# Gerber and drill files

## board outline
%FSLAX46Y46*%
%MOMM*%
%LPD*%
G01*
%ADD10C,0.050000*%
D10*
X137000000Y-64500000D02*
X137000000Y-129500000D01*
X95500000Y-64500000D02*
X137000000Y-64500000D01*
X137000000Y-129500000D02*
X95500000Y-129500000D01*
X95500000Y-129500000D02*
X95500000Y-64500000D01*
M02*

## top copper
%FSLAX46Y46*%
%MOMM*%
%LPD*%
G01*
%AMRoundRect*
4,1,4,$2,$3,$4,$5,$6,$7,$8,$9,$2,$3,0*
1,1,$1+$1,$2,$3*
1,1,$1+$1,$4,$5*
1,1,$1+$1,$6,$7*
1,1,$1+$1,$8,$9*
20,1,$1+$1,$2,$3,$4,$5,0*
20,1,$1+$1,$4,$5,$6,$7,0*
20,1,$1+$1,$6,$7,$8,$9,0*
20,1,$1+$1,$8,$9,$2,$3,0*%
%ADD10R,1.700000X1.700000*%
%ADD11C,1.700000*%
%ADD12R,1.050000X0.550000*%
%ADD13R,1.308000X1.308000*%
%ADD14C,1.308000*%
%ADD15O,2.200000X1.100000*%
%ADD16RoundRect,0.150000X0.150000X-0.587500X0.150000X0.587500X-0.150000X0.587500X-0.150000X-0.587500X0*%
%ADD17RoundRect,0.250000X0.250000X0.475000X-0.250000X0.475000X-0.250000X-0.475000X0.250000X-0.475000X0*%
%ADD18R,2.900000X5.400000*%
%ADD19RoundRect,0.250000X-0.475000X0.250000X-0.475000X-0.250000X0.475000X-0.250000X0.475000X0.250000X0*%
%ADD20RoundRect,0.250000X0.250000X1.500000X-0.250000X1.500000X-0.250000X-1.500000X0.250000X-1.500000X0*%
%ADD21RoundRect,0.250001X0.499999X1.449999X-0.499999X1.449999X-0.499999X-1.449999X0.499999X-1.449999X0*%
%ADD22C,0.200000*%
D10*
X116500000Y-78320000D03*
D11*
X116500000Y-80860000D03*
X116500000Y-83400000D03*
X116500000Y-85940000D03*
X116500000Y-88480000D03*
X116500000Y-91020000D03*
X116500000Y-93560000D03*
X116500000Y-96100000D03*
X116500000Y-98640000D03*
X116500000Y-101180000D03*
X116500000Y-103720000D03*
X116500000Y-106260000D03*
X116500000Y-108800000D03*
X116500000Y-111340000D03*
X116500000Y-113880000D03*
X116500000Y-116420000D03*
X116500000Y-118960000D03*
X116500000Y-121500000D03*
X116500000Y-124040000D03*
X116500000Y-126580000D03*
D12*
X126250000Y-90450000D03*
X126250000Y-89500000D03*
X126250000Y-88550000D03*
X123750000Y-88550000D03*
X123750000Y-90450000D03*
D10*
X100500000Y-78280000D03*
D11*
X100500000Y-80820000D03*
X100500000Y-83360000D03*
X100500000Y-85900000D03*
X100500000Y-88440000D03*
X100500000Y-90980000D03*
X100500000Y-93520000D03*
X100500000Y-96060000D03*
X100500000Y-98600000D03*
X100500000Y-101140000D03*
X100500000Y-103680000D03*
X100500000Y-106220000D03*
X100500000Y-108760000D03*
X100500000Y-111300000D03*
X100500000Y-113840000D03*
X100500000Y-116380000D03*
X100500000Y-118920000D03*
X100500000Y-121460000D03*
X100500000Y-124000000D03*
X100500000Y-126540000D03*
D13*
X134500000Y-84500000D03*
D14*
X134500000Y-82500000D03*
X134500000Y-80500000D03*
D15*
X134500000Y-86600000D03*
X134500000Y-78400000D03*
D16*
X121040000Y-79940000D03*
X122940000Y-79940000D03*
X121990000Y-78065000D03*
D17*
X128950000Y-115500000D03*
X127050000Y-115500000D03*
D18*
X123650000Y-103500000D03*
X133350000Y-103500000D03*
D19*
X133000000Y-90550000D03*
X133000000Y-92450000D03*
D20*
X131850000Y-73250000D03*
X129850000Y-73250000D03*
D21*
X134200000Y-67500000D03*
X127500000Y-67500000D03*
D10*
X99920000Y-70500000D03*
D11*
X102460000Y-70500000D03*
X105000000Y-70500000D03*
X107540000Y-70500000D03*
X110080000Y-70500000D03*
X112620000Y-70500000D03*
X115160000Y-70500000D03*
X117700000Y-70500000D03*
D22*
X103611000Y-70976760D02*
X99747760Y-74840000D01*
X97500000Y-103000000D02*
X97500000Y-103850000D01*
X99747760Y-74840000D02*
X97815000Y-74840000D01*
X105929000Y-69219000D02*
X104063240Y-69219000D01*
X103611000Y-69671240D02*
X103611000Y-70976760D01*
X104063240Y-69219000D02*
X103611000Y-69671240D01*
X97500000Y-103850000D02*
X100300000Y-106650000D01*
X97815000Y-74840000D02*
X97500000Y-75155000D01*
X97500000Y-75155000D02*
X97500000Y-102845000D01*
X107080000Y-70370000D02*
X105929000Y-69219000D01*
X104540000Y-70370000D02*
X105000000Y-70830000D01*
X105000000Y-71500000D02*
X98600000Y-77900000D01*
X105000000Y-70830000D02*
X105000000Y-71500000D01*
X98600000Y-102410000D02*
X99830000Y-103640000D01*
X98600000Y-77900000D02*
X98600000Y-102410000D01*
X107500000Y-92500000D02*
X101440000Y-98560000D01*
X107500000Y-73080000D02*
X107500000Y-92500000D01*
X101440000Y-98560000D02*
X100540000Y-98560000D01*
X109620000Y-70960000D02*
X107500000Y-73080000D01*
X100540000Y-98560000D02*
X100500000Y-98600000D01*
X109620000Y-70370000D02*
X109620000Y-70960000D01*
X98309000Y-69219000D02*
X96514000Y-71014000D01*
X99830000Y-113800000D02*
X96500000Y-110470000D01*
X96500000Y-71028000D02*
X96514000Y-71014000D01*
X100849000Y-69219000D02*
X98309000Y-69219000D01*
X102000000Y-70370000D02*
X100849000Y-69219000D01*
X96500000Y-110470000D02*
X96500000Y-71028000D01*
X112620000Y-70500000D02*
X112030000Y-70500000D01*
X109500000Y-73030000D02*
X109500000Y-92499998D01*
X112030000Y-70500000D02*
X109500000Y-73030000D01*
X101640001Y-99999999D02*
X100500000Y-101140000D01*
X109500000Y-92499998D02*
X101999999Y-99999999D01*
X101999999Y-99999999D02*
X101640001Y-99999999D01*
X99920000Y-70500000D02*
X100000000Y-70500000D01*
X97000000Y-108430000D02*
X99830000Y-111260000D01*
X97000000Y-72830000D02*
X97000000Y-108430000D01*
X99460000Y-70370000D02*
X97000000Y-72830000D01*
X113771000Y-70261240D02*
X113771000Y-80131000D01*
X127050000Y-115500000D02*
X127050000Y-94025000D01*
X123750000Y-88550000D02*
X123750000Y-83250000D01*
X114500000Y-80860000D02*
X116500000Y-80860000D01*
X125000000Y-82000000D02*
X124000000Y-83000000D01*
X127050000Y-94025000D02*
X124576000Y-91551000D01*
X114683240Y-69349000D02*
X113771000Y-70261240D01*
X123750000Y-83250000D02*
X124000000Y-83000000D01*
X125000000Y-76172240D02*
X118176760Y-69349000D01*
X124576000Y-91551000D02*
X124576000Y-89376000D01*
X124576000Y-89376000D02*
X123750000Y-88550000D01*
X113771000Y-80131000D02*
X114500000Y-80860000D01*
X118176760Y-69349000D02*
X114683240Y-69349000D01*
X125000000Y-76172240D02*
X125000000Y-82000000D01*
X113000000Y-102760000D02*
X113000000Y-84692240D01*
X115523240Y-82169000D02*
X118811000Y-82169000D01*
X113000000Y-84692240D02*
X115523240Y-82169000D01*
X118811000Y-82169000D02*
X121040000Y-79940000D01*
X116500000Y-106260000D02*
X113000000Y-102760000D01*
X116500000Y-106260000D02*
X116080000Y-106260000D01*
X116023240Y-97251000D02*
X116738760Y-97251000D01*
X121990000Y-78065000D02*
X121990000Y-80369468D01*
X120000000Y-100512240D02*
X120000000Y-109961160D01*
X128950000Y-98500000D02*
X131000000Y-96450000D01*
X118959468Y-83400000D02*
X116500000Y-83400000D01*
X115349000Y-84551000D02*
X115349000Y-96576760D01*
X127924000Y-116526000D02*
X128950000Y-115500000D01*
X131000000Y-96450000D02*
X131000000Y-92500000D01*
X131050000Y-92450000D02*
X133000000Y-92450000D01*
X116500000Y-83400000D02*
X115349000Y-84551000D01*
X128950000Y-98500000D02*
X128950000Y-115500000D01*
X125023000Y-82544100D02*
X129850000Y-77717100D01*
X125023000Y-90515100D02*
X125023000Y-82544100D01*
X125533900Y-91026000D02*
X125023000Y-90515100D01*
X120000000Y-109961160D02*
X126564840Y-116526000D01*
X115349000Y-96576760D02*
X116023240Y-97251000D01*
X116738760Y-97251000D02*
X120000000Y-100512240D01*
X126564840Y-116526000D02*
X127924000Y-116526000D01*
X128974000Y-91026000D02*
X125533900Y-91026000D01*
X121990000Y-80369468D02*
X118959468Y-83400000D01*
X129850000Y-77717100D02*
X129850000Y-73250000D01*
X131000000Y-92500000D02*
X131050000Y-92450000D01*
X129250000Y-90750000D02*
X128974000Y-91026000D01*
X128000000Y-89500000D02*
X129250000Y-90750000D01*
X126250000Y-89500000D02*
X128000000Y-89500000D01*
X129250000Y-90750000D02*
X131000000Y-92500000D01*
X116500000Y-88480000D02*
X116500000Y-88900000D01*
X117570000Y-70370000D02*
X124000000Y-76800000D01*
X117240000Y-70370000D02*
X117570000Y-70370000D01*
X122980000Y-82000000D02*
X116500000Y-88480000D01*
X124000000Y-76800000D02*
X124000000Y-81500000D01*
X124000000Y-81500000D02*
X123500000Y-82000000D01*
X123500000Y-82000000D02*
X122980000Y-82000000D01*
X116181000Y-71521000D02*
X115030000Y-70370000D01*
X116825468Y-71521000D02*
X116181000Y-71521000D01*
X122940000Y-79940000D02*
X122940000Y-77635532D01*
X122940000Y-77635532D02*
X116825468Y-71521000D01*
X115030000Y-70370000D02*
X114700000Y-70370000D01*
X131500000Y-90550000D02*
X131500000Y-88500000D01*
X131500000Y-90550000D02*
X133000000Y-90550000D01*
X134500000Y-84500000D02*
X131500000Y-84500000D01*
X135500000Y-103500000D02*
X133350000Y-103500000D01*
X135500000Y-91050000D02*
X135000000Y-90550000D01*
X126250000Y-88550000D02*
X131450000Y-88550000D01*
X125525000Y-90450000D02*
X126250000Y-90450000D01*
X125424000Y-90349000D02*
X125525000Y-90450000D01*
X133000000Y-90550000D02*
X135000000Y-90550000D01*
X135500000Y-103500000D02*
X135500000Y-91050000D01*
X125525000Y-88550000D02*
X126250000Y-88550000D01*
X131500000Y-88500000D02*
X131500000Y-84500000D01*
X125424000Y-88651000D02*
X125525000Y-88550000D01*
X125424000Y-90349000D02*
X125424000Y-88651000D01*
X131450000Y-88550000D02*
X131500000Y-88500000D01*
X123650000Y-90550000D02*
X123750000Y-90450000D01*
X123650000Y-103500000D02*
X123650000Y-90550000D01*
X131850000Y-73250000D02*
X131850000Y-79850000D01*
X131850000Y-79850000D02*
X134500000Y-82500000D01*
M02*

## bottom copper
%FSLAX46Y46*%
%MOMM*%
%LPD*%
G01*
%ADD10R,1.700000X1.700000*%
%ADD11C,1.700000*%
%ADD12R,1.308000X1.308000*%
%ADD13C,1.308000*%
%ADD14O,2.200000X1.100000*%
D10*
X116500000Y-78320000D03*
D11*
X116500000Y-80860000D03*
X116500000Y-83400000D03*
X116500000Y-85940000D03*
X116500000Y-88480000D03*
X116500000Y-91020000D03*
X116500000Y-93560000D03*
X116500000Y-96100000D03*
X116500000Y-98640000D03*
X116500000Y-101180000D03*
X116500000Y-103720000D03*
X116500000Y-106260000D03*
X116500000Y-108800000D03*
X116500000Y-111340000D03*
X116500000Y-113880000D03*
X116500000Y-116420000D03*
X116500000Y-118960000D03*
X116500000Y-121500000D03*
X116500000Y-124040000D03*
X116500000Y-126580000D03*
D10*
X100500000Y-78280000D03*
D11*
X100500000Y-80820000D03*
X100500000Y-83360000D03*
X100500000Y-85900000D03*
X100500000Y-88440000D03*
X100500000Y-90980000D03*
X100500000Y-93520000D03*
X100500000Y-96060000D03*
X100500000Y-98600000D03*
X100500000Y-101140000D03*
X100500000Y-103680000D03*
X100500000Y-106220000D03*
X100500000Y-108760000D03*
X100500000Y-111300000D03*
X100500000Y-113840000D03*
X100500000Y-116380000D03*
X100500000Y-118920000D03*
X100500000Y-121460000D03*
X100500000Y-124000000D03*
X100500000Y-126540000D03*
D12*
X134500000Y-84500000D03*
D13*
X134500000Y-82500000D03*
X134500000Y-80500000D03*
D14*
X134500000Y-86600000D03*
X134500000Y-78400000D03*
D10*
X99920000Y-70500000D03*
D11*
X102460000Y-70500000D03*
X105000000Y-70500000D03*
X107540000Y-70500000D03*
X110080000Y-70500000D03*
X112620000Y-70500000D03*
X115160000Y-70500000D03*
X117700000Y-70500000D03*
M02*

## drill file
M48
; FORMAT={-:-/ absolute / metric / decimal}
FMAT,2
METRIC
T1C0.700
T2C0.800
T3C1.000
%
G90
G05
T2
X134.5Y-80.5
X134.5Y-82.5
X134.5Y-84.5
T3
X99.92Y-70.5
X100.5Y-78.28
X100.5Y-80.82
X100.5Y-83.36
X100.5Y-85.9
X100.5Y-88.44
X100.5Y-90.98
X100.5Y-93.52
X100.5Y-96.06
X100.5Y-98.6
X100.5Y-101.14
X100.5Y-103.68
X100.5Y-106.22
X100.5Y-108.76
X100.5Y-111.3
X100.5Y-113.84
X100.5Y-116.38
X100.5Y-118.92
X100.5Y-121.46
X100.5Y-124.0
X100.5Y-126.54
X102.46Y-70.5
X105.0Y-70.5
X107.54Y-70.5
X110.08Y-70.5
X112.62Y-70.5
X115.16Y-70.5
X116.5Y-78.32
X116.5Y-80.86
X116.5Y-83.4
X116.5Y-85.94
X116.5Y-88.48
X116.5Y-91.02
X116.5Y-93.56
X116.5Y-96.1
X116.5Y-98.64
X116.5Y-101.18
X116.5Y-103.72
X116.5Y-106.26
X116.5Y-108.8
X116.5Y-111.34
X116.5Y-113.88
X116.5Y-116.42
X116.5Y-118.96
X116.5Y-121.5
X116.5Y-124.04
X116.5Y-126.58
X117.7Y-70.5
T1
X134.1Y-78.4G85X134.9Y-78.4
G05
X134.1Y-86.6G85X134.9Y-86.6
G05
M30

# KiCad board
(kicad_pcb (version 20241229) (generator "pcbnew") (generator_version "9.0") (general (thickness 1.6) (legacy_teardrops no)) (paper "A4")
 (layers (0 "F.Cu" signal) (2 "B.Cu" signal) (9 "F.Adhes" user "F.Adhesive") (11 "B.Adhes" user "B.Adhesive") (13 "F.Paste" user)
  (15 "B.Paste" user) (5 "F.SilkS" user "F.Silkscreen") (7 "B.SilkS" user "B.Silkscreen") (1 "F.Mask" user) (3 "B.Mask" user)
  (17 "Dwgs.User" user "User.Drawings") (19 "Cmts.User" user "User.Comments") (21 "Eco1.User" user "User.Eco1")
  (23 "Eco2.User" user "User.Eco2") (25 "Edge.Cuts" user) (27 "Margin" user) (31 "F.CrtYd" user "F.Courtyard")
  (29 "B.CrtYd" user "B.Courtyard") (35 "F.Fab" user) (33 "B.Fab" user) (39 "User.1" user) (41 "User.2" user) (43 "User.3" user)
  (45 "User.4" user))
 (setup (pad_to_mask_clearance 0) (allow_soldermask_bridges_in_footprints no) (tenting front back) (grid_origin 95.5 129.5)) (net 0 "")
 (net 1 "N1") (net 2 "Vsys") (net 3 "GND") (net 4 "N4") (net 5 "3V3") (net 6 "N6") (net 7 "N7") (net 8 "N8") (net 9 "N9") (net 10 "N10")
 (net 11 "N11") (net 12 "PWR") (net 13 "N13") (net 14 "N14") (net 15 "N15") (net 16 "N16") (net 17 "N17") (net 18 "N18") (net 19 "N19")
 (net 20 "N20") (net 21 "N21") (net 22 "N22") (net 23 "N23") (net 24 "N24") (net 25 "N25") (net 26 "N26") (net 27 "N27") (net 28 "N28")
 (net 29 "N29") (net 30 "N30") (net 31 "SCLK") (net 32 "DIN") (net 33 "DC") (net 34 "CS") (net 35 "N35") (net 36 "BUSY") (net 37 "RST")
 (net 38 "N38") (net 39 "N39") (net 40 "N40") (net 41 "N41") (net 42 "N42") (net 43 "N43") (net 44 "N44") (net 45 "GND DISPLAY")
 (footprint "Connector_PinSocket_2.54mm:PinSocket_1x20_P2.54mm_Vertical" (layer "F.Cu") (at 116.5 78.32)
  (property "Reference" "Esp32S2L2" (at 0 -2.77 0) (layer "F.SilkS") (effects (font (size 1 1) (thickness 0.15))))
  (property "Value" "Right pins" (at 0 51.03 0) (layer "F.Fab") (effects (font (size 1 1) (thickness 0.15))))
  (pad "1" thru_hole rect (at 0 0) (size 1.7 1.7) (drill 1) (layers "*.Cu" "*.Mask") (remove_unused_layers no) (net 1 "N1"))
  (pad "2" thru_hole circle (at 0 2.54) (size 1.7 1.7) (drill 1) (layers "*.Cu" "*.Mask") (remove_unused_layers no) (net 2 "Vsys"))
  (pad "3" thru_hole circle (at 0 5.08) (size 1.7 1.7) (drill 1) (layers "*.Cu" "*.Mask") (remove_unused_layers no) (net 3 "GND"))
  (pad "4" thru_hole circle (at 0 7.62) (size 1.7 1.7) (drill 1) (layers "*.Cu" "*.Mask") (remove_unused_layers no) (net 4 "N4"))
  (pad "5" thru_hole circle (at 0 10.16) (size 1.7 1.7) (drill 1) (layers "*.Cu" "*.Mask") (remove_unused_layers no) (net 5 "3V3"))
  (pad "6" thru_hole circle (at 0 12.7) (size 1.7 1.7) (drill 1) (layers "*.Cu" "*.Mask") (remove_unused_layers no) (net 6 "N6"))
  (pad "7" thru_hole circle (at 0 15.24) (size 1.7 1.7) (drill 1) (layers "*.Cu" "*.Mask") (remove_unused_layers no) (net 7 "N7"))
  (pad "8" thru_hole circle (at 0 17.78) (size 1.7 1.7) (drill 1) (layers "*.Cu" "*.Mask") (remove_unused_layers no) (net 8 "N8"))
  (pad "9" thru_hole circle (at 0 20.32) (size 1.7 1.7) (drill 1) (layers "*.Cu" "*.Mask") (remove_unused_layers no) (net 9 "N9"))
  (pad "10" thru_hole circle (at 0 22.86) (size 1.7 1.7) (drill 1) (layers "*.Cu" "*.Mask") (remove_unused_layers no) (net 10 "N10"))
  (pad "11" thru_hole circle (at 0 25.4) (size 1.7 1.7) (drill 1) (layers "*.Cu" "*.Mask") (remove_unused_layers no) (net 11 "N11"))
  (pad "12" thru_hole circle (at 0 27.94) (size 1.7 1.7) (drill 1) (layers "*.Cu" "*.Mask") (remove_unused_layers no) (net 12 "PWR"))
  (pad "13" thru_hole circle (at 0 30.48) (size 1.7 1.7) (drill 1) (layers "*.Cu" "*.Mask") (remove_unused_layers no) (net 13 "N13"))
  (pad "14" thru_hole circle (at 0 33.02) (size 1.7 1.7) (drill 1) (layers "*.Cu" "*.Mask") (remove_unused_layers no) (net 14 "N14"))
  (pad "15" thru_hole circle (at 0 35.56) (size 1.7 1.7) (drill 1) (layers "*.Cu" "*.Mask") (remove_unused_layers no) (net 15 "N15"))
  (pad "16" thru_hole circle (at 0 38.1) (size 1.7 1.7) (drill 1) (layers "*.Cu" "*.Mask") (remove_unused_layers no) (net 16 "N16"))
  (pad "17" thru_hole circle (at 0 40.64) (size 1.7 1.7) (drill 1) (layers "*.Cu" "*.Mask") (remove_unused_layers no) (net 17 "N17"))
  (pad "18" thru_hole circle (at 0 43.18) (size 1.7 1.7) (drill 1) (layers "*.Cu" "*.Mask") (remove_unused_layers no) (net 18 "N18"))
  (pad "19" thru_hole circle (at 0 45.72) (size 1.7 1.7) (drill 1) (layers "*.Cu" "*.Mask") (remove_unused_layers no) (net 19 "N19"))
  (pad "20" thru_hole circle (at 0 48.26) (size 1.7 1.7) (drill 1) (layers "*.Cu" "*.Mask") (remove_unused_layers no) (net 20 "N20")))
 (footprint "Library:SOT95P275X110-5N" (layer "F.Cu") (at 125 89.5 180)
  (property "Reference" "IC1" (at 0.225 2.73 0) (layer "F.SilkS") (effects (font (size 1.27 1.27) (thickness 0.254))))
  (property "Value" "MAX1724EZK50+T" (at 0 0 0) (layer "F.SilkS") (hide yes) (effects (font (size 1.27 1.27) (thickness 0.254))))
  (pad "1" smd rect (at -1.25 -0.95 270) (size 0.55 1.05) (layers "F.Cu" "F.Mask" "F.Paste") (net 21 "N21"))
  (pad "2" smd rect (at -1.25 0 270) (size 0.55 1.05) (layers "F.Cu" "F.Mask" "F.Paste") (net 3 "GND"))
  (pad "3" smd rect (at -1.25 0.95 270) (size 0.55 1.05) (layers "F.Cu" "F.Mask" "F.Paste") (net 21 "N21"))
  (pad "4" smd rect (at 1.25 0.95 270) (size 0.55 1.05) (layers "F.Cu" "F.Mask" "F.Paste") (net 2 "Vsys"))
  (pad "5" smd rect (at 1.25 -0.95 270) (size 0.55 1.05) (layers "F.Cu" "F.Mask" "F.Paste") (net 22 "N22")))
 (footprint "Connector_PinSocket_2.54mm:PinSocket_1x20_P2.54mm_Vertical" (layer "F.Cu") (at 100.5 78.28)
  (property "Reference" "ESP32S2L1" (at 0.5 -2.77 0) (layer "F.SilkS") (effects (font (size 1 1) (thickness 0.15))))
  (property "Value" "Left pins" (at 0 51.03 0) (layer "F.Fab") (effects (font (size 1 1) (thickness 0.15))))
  (pad "1" thru_hole rect (at 0 0) (size 1.7 1.7) (drill 1) (layers "*.Cu" "*.Mask") (remove_unused_layers no) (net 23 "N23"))
  (pad "2" thru_hole circle (at 0 2.54) (size 1.7 1.7) (drill 1) (layers "*.Cu" "*.Mask") (remove_unused_layers no) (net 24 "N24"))
  (pad "3" thru_hole circle (at 0 5.08) (size 1.7 1.7) (drill 1) (layers "*.Cu" "*.Mask") (remove_unused_layers no) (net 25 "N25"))
  (pad "4" thru_hole circle (at 0 7.62) (size 1.7 1.7) (drill 1) (layers "*.Cu" "*.Mask") (remove_unused_layers no) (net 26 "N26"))
  (pad "5" thru_hole circle (at 0 10.16) (size 1.7 1.7) (drill 1) (layers "*.Cu" "*.Mask") (remove_unused_layers no) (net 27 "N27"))
  (pad "6" thru_hole circle (at 0 12.7) (size 1.7 1.7) (drill 1) (layers "*.Cu" "*.Mask") (remove_unused_layers no) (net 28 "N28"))
  (pad "7" thru_hole circle (at 0 15.24) (size 1.7 1.7) (drill 1) (layers "*.Cu" "*.Mask") (remove_unused_layers no) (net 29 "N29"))
  (pad "8" thru_hole circle (at 0 17.78) (size 1.7 1.7) (drill 1) (layers "*.Cu" "*.Mask") (remove_unused_layers no) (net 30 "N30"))
  (pad "9" thru_hole circle (at 0 20.32) (size 1.7 1.7) (drill 1) (layers "*.Cu" "*.Mask") (remove_unused_layers no) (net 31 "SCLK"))
  (pad "10" thru_hole circle (at 0 22.86) (size 1.7 1.7) (drill 1) (layers "*.Cu" "*.Mask") (remove_unused_layers no) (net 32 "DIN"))
  (pad "11" thru_hole circle (at 0 25.4) (size 1.7 1.7) (drill 1) (layers "*.Cu" "*.Mask") (remove_unused_layers no) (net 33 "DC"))
  (pad "12" thru_hole circle (at 0 27.94) (size 1.7 1.7) (drill 1) (layers "*.Cu" "*.Mask") (remove_unused_layers no) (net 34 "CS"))
  (pad "13" thru_hole circle (at 0 30.48) (size 1.7 1.7) (drill 1) (layers "*.Cu" "*.Mask") (remove_unused_layers no) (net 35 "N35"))
  (pad "14" thru_hole circle (at 0 33.02) (size 1.7 1.7) (drill 1) (layers "*.Cu" "*.Mask") (remove_unused_layers no) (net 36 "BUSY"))
  (pad "15" thru_hole circle (at 0 35.56) (size 1.7 1.7) (drill 1) (layers "*.Cu" "*.Mask") (remove_unused_layers no) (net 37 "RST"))
  (pad "16" thru_hole circle (at 0 38.1) (size 1.7 1.7) (drill 1) (layers "*.Cu" "*.Mask") (remove_unused_layers no) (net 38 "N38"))
  (pad "17" thru_hole circle (at 0 40.64) (size 1.7 1.7) (drill 1) (layers "*.Cu" "*.Mask") (remove_unused_layers no) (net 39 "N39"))
  (pad "18" thru_hole circle (at 0 43.18) (size 1.7 1.7) (drill 1) (layers "*.Cu" "*.Mask") (remove_unused_layers no) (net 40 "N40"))
  (pad "19" thru_hole circle (at 0 45.72) (size 1.7 1.7) (drill 1) (layers "*.Cu" "*.Mask") (remove_unused_layers no) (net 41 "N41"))
  (pad "20" thru_hole circle (at 0 48.26) (size 1.7 1.7) (drill 1) (layers "*.Cu" "*.Mask") (remove_unused_layers no) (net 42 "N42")))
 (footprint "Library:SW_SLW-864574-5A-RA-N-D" (layer "F.Cu") (at 134.5 82.5 90)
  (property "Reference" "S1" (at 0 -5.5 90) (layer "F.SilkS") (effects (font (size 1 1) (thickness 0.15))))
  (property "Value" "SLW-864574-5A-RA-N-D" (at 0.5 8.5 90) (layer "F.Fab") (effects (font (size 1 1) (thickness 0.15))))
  (pad "1" thru_hole rect (at -2 0 90) (size 1.308 1.308) (drill 0.8) (layers "*.Cu" "*.Mask") (remove_unused_layers no) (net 21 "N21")
   (solder_mask_margin 0.102))
  (pad "2" thru_hole circle (at 0 0 90) (size 1.308 1.308) (drill 0.8) (layers "*.Cu" "*.Mask") (remove_unused_layers no) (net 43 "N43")
   (solder_mask_margin 0.102))
  (pad "3" thru_hole circle (at 2 0 90) (size 1.308 1.308) (drill 0.8) (layers "*.Cu" "*.Mask") (remove_unused_layers no) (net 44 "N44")
   (solder_mask_margin 0.102))
  (pad "SH1" thru_hole oval (at -4.1 0 90) (size 1.1 2.2) (drill oval 0.7 1.5) (layers "*.Cu" "*.Mask") (remove_unused_layers no)
   (solder_mask_margin 0.102))
  (pad "SH2" thru_hole oval (at 4.1 0 90) (size 1.1 2.2) (drill oval 0.7 1.5) (layers "*.Cu" "*.Mask") (remove_unused_layers no)
   (solder_mask_margin 0.102)))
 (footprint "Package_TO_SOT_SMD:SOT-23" (layer "F.Cu") (at 121.99 79.0025 90)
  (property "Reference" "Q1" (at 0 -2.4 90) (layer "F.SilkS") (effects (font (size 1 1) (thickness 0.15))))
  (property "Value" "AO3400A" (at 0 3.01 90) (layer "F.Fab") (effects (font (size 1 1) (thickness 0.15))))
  (pad "1" smd roundrect (at -0.9375 -0.95 90) (size 1.475 0.6) (layers "F.Cu" "F.Mask" "F.Paste") (roundrect_rratio 0.25) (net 12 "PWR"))
  (pad "2" smd roundrect (at -0.9375 0.95 90) (size 1.475 0.6) (layers "F.Cu" "F.Mask" "F.Paste") (roundrect_rratio 0.25)
   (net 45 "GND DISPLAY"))
  (pad "3" smd roundrect (at 0.9375 0 90) (size 1.475 0.6) (layers "F.Cu" "F.Mask" "F.Paste") (roundrect_rratio 0.25) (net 3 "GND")))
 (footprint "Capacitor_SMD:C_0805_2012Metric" (layer "F.Cu") (at 128 115.5 180)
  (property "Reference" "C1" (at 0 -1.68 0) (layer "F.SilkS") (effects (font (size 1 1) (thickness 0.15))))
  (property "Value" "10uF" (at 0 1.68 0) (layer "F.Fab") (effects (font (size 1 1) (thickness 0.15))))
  (pad "1" smd roundrect (at -0.95 0 180) (size 1 1.45) (layers "F.Cu" "F.Mask" "F.Paste") (roundrect_rratio 0.25) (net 3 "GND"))
  (pad "2" smd roundrect (at 0.95 0 180) (size 1 1.45) (layers "F.Cu" "F.Mask" "F.Paste") (roundrect_rratio 0.25) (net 2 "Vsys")))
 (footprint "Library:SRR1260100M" (layer "F.Cu") (at 128.5 103.5)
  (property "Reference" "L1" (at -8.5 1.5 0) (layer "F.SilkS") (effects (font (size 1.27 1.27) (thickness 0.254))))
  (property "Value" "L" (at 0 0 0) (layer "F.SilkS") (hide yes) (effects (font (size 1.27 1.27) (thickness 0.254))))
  (pad "1" smd rect (at -4.85 0) (size 2.9 5.4) (layers "F.Cu" "F.Mask" "F.Paste") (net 22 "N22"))
  (pad "2" smd rect (at 4.85 0) (size 2.9 5.4) (layers "F.Cu" "F.Mask" "F.Paste") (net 21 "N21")))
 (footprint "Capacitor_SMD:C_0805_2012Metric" (layer "F.Cu") (at 133 91.5 -90)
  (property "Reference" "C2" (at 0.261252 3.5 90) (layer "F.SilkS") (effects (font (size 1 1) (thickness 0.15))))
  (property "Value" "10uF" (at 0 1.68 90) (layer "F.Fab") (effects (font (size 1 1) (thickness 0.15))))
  (pad "1" smd roundrect (at -0.95 0 270) (size 1 1.45) (layers "F.Cu" "F.Mask" "F.Paste") (roundrect_rratio 0.25) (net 21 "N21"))
  (pad "2" smd roundrect (at 0.95 0 270) (size 1 1.45) (layers "F.Cu" "F.Mask" "F.Paste") (roundrect_rratio 0.25) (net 3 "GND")))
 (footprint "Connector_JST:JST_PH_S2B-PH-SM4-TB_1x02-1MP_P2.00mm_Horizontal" (layer "F.Cu") (at 130.85 70.4 180)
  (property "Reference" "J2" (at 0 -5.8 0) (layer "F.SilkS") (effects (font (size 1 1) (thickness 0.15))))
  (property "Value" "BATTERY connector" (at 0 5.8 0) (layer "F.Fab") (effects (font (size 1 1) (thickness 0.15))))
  (pad "1" smd roundrect (at -1 -2.85 180) (size 1 3.5) (layers "F.Cu" "F.Mask" "F.Paste") (roundrect_rratio 0.25) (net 43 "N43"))
  (pad "2" smd roundrect (at 1 -2.85 180) (size 1 3.5) (layers "F.Cu" "F.Mask" "F.Paste") (roundrect_rratio 0.25) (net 3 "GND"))
  (pad "MP" smd roundrect (at -3.35 2.9 180) (size 1.5 3.4) (layers "F.Cu" "F.Mask" "F.Paste") (roundrect_rratio 0.166667))
  (pad "MP" smd roundrect (at 3.35 2.9 180) (size 1.5 3.4) (layers "F.Cu" "F.Mask" "F.Paste") (roundrect_rratio 0.166667)))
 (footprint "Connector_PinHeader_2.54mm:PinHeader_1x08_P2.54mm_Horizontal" (layer "F.Cu") (at 99.92 70.5 90)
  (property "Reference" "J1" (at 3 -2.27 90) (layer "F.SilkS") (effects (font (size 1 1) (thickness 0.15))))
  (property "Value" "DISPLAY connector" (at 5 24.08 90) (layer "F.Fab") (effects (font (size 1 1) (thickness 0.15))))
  (pad "1" thru_hole rect (at 0 0 90) (size 1.7 1.7) (drill 1) (layers "*.Cu" "*.Mask") (remove_unused_layers no) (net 36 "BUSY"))
  (pad "2" thru_hole circle (at 0 2.54 90) (size 1.7 1.7) (drill 1) (layers "*.Cu" "*.Mask") (remove_unused_layers no) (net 37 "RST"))
  (pad "3" thru_hole circle (at 0 5.08 90) (size 1.7 1.7) (drill 1) (layers "*.Cu" "*.Mask") (remove_unused_layers no) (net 33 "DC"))
  (pad "4" thru_hole circle (at 0 7.62 90) (size 1.7 1.7) (drill 1) (layers "*.Cu" "*.Mask") (remove_unused_layers no) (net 34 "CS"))
  (pad "5" thru_hole circle (at 0 10.16 90) (size 1.7 1.7) (drill 1) (layers "*.Cu" "*.Mask") (remove_unused_layers no) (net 31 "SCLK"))
  (pad "6" thru_hole circle (at 0 12.7 90) (size 1.7 1.7) (drill 1) (layers "*.Cu" "*.Mask") (remove_unused_layers no) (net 32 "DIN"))
  (pad "7" thru_hole circle (at 0 15.24 90) (size 1.7 1.7) (drill 1) (layers "*.Cu" "*.Mask") (remove_unused_layers no)
   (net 45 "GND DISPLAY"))
  (pad "8" thru_hole circle (at 0 17.78 90) (size 1.7 1.7) (drill 1) (layers "*.Cu" "*.Mask") (remove_unused_layers no) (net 5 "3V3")))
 (gr_line (start 137 64.5) (end 137 129.5) (stroke (width 0.05) (type default)) (layer "Edge.Cuts"))
 (gr_line (start 95.5 64.5) (end 137 64.5) (stroke (width 0.05) (type default)) (layer "Edge.Cuts"))
 (gr_line (start 137 129.5) (end 95.5 129.5) (stroke (width 0.05) (type default)) (layer "Edge.Cuts"))
 (gr_line (start 95.5 129.5) (end 95.5 64.5) (stroke (width 0.05) (type default)) (layer "Edge.Cuts"))
 (segment (start 103.611 70.97676) (end 99.74776 74.84) (width 0.2) (layer "F.Cu") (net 34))
 (segment (start 97.5 103) (end 97.5 103.85) (width 0.2) (layer "F.Cu") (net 34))
 (segment (start 99.74776 74.84) (end 97.815 74.84) (width 0.2) (layer "F.Cu") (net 34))
 (segment (start 105.929 69.219) (end 104.06324 69.219) (width 0.2) (layer "F.Cu") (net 34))
 (segment (start 103.611 69.67124) (end 103.611 70.97676) (width 0.2) (layer "F.Cu") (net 34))
 (segment (start 104.06324 69.219) (end 103.611 69.67124) (width 0.2) (layer "F.Cu") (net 34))
 (segment (start 97.5 103.85) (end 100.3 106.65) (width 0.2) (layer "F.Cu") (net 34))
 (segment (start 97.815 74.84) (end 97.5 75.155) (width 0.2) (layer "F.Cu") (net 34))
 (segment (start 97.5 75.155) (end 97.5 102.845) (width 0.2) (layer "F.Cu") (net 34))
 (segment (start 107.08 70.37) (end 105.929 69.219) (width 0.2) (layer "F.Cu") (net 34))
 (segment (start 104.54 70.37) (end 105 70.83) (width 0.2) (layer "F.Cu") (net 33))
 (segment (start 105 71.5) (end 98.6 77.9) (width 0.2) (layer "F.Cu") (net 33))
 (segment (start 105 70.83) (end 105 71.5) (width 0.2) (layer "F.Cu") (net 33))
 (segment (start 98.6 102.41) (end 99.83 103.64) (width 0.2) (layer "F.Cu") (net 33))
 (segment (start 98.6 77.9) (end 98.6 102.41) (width 0.2) (layer "F.Cu") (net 33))
 (segment (start 107.5 92.5) (end 101.44 98.56) (width 0.2) (layer "F.Cu") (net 31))
 (segment (start 107.5 73.08) (end 107.5 92.5) (width 0.2) (layer "F.Cu") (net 31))
 (segment (start 101.44 98.56) (end 100.54 98.56) (width 0.2) (layer "F.Cu") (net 31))
 (segment (start 109.62 70.96) (end 107.5 73.08) (width 0.2) (layer "F.Cu") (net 31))
 (segment (start 100.54 98.56) (end 100.5 98.6) (width 0.2) (layer "F.Cu") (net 31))
 (segment (start 109.62 70.37) (end 109.62 70.96) (width 0.2) (layer "F.Cu") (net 31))
 (segment (start 98.309 69.219) (end 96.514 71.014) (width 0.2) (layer "F.Cu") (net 37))
 (segment (start 99.83 113.8) (end 96.5 110.47) (width 0.2) (layer "F.Cu") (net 37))
 (segment (start 96.5 71.028) (end 96.514 71.014) (width 0.2) (layer "F.Cu") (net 37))
 (segment (start 100.849 69.219) (end 98.309 69.219) (width 0.2) (layer "F.Cu") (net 37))
 (segment (start 102 70.37) (end 100.849 69.219) (width 0.2) (layer "F.Cu") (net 37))
 (segment (start 96.5 110.47) (end 96.5 71.028) (width 0.2) (layer "F.Cu") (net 37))
 (segment (start 112.62 70.5) (end 112.03 70.5) (width 0.2) (layer "F.Cu") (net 32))
 (segment (start 109.5 73.03) (end 109.5 92.499998) (width 0.2) (layer "F.Cu") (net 32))
 (segment (start 112.03 70.5) (end 109.5 73.03) (width 0.2) (layer "F.Cu") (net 32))
 (segment (start 101.640001 99.999999) (end 100.5 101.14) (width 0.2) (layer "F.Cu") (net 32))
 (segment (start 109.5 92.499998) (end 101.999999 99.999999) (width 0.2) (layer "F.Cu") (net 32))
 (segment (start 101.999999 99.999999) (end 101.640001 99.999999) (width 0.2) (layer "F.Cu") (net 32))
 (segment (start 99.92 70.5) (end 100 70.5) (width 0.2) (layer "F.Cu") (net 36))
 (segment (start 97 108.43) (end 99.83 111.26) (width 0.2) (layer "F.Cu") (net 36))
 (segment (start 97 72.83) (end 97 108.43) (width 0.2) (layer "F.Cu") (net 36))
 (segment (start 99.46 70.37) (end 97 72.83) (width 0.2) (layer "F.Cu") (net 36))
 (segment (start 113.771 70.26124) (end 113.771 80.131) (width 0.2) (layer "F.Cu") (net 2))
 (segment (start 127.05 115.5) (end 127.05 94.025) (width 0.2) (layer "F.Cu") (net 2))
 (segment (start 123.75 88.55) (end 123.75 83.25) (width 0.2) (layer "F.Cu") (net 2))
 (segment (start 114.5 80.86) (end 116.5 80.86) (width 0.2) (layer "F.Cu") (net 2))
 (segment (start 125 82) (end 124 83) (width 0.2) (layer "F.Cu") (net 2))
 (segment (start 127.05 94.025) (end 124.576 91.551) (width 0.2) (layer "F.Cu") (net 2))
 (segment (start 114.68324 69.349) (end 113.771 70.26124) (width 0.2) (layer "F.Cu") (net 2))
 (segment (start 123.75 83.25) (end 124 83) (width 0.2) (layer "F.Cu") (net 2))
 (segment (start 125 76.17224) (end 118.17676 69.349) (width 0.2) (layer "F.Cu") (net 2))
 (segment (start 124.576 91.551) (end 124.576 89.376) (width 0.2) (layer "F.Cu") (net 2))
 (segment (start 124.576 89.376) (end 123.75 88.55) (width 0.2) (layer "F.Cu") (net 2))
 (segment (start 113.771 80.131) (end 114.5 80.86) (width 0.2) (layer "F.Cu") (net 2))
 (segment (start 118.17676 69.349) (end 114.68324 69.349) (width 0.2) (layer "F.Cu") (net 2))
 (segment (start 125 76.17224) (end 125 82) (width 0.2) (layer "F.Cu") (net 2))
 (segment (start 113 102.76) (end 113 84.69224) (width 0.2) (layer "F.Cu") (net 12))
 (segment (start 115.52324 82.169) (end 118.811 82.169) (width 0.2) (layer "F.Cu") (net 12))
 (segment (start 113 84.69224) (end 115.52324 82.169) (width 0.2) (layer "F.Cu") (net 12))
 (segment (start 118.811 82.169) (end 121.04 79.94) (width 0.2) (layer "F.Cu") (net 12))
 (segment (start 116.5 106.26) (end 113 102.76) (width 0.2) (layer "F.Cu") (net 12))
 (segment (start 116.5 106.26) (end 116.08 106.26) (width 0.2) (layer "F.Cu") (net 12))
 (segment (start 116.02324 97.251) (end 116.73876 97.251) (width 0.2) (layer "F.Cu") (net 3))
 (segment (start 121.99 78.065) (end 121.99 80.369468) (width 0.2) (layer "F.Cu") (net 3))
 (segment (start 120 100.51224) (end 120 109.96116) (width 0.2) (layer "F.Cu") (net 3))
 (segment (start 128.95 98.5) (end 131 96.45) (width 0.2) (layer "F.Cu") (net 3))
 (segment (start 118.959468 83.4) (end 116.5 83.4) (width 0.2) (layer "F.Cu") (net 3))
 (segment (start 115.349 84.551) (end 115.349 96.57676) (width 0.2) (layer "F.Cu") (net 3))
 (segment (start 127.924 116.526) (end 128.95 115.5) (width 0.2) (layer "F.Cu") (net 3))
 (segment (start 131 96.45) (end 131 92.5) (width 0.2) (layer "F.Cu") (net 3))
 (segment (start 131.05 92.45) (end 133 92.45) (width 0.2) (layer "F.Cu") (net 3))
 (segment (start 116.5 83.4) (end 115.349 84.551) (width 0.2) (layer "F.Cu") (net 3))
 (segment (start 128.95 98.5) (end 128.95 115.5) (width 0.2) (layer "F.Cu") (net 3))
 (segment (start 125.023 82.5441) (end 129.85 77.7171) (width 0.2) (layer "F.Cu") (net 3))
 (segment (start 125.023 90.5151) (end 125.023 82.5441) (width 0.2) (layer "F.Cu") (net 3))
 (segment (start 125.5339 91.026) (end 125.023 90.5151) (width 0.2) (layer "F.Cu") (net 3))
 (segment (start 120 109.96116) (end 126.56484 116.526) (width 0.2) (layer "F.Cu") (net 3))
 (segment (start 115.349 96.57676) (end 116.02324 97.251) (width 0.2) (layer "F.Cu") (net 3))
 (segment (start 116.73876 97.251) (end 120 100.51224) (width 0.2) (layer "F.Cu") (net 3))
 (segment (start 126.56484 116.526) (end 127.924 116.526) (width 0.2) (layer "F.Cu") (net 3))
 (segment (start 128.974 91.026) (end 125.5339 91.026) (width 0.2) (layer "F.Cu") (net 3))
 (segment (start 121.99 80.369468) (end 118.959468 83.4) (width 0.2) (layer "F.Cu") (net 3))
 (segment (start 129.85 77.7171) (end 129.85 73.25) (width 0.2) (layer "F.Cu") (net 3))
 (segment (start 131 92.5) (end 131.05 92.45) (width 0.2) (layer "F.Cu") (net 3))
 (segment (start 129.25 90.75) (end 128.974 91.026) (width 0.2) (layer "F.Cu") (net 3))
 (segment (start 128 89.5) (end 129.25 90.75) (width 0.2) (layer "F.Cu") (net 3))
 (segment (start 126.25 89.5) (end 128 89.5) (width 0.2) (layer "F.Cu") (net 3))
 (segment (start 129.25 90.75) (end 131 92.5) (width 0.2) (layer "F.Cu") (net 3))
 (segment (start 116.5 88.48) (end 116.5 88.9) (width 0.2) (layer "F.Cu") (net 5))
 (segment (start 117.57 70.37) (end 124 76.8) (width 0.2) (layer "F.Cu") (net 5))
 (segment (start 117.24 70.37) (end 117.57 70.37) (width 0.2) (layer "F.Cu") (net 5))
 (segment (start 122.98 82) (end 116.5 88.48) (width 0.2) (layer "F.Cu") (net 5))
 (segment (start 124 76.8) (end 124 81.5) (width 0.2) (layer "F.Cu") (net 5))
 (segment (start 124 81.5) (end 123.5 82) (width 0.2) (layer "F.Cu") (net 5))
 (segment (start 123.5 82) (end 122.98 82) (width 0.2) (layer "F.Cu") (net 5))
 (segment (start 116.181 71.521) (end 115.03 70.37) (width 0.2) (layer "F.Cu") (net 45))
 (segment (start 116.825468 71.521) (end 116.181 71.521) (width 0.2) (layer "F.Cu") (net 45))
 (segment (start 122.94 79.94) (end 122.94 77.635532) (width 0.2) (layer "F.Cu") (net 45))
 (segment (start 122.94 77.635532) (end 116.825468 71.521) (width 0.2) (layer "F.Cu") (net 45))
 (segment (start 115.03 70.37) (end 114.7 70.37) (width 0.2) (layer "F.Cu") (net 45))
 (segment (start 131.5 90.55) (end 131.5 88.5) (width 0.2) (layer "F.Cu") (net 21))
 (segment (start 131.5 90.55) (end 133 90.55) (width 0.2) (layer "F.Cu") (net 21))
 (segment (start 134.5 84.5) (end 131.5 84.5) (width 0.2) (layer "F.Cu") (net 21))
 (segment (start 135.5 103.5) (end 133.35 103.5) (width 0.2) (layer "F.Cu") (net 21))
 (segment (start 135.5 91.05) (end 135 90.55) (width 0.2) (layer "F.Cu") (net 21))
 (segment (start 126.25 88.55) (end 131.45 88.55) (width 0.2) (layer "F.Cu") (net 21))
 (segment (start 125.525 90.45) (end 126.25 90.45) (width 0.2) (layer "F.Cu") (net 21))
 (segment (start 125.424 90.349) (end 125.525 90.45) (width 0.2) (layer "F.Cu") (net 21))
 (segment (start 133 90.55) (end 135 90.55) (width 0.2) (layer "F.Cu") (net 21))
 (segment (start 135.5 103.5) (end 135.5 91.05) (width 0.2) (layer "F.Cu") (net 21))
 (segment (start 125.525 88.55) (end 126.25 88.55) (width 0.2) (layer "F.Cu") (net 21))
 (segment (start 131.5 88.5) (end 131.5 84.5) (width 0.2) (layer "F.Cu") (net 21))
 (segment (start 125.424 88.651) (end 125.525 88.55) (width 0.2) (layer "F.Cu") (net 21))
 (segment (start 125.424 90.349) (end 125.424 88.651) (width 0.2) (layer "F.Cu") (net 21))
 (segment (start 131.45 88.55) (end 131.5 88.5) (width 0.2) (layer "F.Cu") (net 21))
 (segment (start 123.65 90.55) (end 123.75 90.45) (width 0.2) (layer "F.Cu") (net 22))
 (segment (start 123.65 103.5) (end 123.65 90.55) (width 0.2) (layer "F.Cu") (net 22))
 (segment (start 131.85 73.25) (end 131.85 79.85) (width 0.2) (layer "F.Cu") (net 43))
 (segment (start 131.85 79.85) (end 134.5 82.5) (width 0.2) (layer "F.Cu") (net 43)))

